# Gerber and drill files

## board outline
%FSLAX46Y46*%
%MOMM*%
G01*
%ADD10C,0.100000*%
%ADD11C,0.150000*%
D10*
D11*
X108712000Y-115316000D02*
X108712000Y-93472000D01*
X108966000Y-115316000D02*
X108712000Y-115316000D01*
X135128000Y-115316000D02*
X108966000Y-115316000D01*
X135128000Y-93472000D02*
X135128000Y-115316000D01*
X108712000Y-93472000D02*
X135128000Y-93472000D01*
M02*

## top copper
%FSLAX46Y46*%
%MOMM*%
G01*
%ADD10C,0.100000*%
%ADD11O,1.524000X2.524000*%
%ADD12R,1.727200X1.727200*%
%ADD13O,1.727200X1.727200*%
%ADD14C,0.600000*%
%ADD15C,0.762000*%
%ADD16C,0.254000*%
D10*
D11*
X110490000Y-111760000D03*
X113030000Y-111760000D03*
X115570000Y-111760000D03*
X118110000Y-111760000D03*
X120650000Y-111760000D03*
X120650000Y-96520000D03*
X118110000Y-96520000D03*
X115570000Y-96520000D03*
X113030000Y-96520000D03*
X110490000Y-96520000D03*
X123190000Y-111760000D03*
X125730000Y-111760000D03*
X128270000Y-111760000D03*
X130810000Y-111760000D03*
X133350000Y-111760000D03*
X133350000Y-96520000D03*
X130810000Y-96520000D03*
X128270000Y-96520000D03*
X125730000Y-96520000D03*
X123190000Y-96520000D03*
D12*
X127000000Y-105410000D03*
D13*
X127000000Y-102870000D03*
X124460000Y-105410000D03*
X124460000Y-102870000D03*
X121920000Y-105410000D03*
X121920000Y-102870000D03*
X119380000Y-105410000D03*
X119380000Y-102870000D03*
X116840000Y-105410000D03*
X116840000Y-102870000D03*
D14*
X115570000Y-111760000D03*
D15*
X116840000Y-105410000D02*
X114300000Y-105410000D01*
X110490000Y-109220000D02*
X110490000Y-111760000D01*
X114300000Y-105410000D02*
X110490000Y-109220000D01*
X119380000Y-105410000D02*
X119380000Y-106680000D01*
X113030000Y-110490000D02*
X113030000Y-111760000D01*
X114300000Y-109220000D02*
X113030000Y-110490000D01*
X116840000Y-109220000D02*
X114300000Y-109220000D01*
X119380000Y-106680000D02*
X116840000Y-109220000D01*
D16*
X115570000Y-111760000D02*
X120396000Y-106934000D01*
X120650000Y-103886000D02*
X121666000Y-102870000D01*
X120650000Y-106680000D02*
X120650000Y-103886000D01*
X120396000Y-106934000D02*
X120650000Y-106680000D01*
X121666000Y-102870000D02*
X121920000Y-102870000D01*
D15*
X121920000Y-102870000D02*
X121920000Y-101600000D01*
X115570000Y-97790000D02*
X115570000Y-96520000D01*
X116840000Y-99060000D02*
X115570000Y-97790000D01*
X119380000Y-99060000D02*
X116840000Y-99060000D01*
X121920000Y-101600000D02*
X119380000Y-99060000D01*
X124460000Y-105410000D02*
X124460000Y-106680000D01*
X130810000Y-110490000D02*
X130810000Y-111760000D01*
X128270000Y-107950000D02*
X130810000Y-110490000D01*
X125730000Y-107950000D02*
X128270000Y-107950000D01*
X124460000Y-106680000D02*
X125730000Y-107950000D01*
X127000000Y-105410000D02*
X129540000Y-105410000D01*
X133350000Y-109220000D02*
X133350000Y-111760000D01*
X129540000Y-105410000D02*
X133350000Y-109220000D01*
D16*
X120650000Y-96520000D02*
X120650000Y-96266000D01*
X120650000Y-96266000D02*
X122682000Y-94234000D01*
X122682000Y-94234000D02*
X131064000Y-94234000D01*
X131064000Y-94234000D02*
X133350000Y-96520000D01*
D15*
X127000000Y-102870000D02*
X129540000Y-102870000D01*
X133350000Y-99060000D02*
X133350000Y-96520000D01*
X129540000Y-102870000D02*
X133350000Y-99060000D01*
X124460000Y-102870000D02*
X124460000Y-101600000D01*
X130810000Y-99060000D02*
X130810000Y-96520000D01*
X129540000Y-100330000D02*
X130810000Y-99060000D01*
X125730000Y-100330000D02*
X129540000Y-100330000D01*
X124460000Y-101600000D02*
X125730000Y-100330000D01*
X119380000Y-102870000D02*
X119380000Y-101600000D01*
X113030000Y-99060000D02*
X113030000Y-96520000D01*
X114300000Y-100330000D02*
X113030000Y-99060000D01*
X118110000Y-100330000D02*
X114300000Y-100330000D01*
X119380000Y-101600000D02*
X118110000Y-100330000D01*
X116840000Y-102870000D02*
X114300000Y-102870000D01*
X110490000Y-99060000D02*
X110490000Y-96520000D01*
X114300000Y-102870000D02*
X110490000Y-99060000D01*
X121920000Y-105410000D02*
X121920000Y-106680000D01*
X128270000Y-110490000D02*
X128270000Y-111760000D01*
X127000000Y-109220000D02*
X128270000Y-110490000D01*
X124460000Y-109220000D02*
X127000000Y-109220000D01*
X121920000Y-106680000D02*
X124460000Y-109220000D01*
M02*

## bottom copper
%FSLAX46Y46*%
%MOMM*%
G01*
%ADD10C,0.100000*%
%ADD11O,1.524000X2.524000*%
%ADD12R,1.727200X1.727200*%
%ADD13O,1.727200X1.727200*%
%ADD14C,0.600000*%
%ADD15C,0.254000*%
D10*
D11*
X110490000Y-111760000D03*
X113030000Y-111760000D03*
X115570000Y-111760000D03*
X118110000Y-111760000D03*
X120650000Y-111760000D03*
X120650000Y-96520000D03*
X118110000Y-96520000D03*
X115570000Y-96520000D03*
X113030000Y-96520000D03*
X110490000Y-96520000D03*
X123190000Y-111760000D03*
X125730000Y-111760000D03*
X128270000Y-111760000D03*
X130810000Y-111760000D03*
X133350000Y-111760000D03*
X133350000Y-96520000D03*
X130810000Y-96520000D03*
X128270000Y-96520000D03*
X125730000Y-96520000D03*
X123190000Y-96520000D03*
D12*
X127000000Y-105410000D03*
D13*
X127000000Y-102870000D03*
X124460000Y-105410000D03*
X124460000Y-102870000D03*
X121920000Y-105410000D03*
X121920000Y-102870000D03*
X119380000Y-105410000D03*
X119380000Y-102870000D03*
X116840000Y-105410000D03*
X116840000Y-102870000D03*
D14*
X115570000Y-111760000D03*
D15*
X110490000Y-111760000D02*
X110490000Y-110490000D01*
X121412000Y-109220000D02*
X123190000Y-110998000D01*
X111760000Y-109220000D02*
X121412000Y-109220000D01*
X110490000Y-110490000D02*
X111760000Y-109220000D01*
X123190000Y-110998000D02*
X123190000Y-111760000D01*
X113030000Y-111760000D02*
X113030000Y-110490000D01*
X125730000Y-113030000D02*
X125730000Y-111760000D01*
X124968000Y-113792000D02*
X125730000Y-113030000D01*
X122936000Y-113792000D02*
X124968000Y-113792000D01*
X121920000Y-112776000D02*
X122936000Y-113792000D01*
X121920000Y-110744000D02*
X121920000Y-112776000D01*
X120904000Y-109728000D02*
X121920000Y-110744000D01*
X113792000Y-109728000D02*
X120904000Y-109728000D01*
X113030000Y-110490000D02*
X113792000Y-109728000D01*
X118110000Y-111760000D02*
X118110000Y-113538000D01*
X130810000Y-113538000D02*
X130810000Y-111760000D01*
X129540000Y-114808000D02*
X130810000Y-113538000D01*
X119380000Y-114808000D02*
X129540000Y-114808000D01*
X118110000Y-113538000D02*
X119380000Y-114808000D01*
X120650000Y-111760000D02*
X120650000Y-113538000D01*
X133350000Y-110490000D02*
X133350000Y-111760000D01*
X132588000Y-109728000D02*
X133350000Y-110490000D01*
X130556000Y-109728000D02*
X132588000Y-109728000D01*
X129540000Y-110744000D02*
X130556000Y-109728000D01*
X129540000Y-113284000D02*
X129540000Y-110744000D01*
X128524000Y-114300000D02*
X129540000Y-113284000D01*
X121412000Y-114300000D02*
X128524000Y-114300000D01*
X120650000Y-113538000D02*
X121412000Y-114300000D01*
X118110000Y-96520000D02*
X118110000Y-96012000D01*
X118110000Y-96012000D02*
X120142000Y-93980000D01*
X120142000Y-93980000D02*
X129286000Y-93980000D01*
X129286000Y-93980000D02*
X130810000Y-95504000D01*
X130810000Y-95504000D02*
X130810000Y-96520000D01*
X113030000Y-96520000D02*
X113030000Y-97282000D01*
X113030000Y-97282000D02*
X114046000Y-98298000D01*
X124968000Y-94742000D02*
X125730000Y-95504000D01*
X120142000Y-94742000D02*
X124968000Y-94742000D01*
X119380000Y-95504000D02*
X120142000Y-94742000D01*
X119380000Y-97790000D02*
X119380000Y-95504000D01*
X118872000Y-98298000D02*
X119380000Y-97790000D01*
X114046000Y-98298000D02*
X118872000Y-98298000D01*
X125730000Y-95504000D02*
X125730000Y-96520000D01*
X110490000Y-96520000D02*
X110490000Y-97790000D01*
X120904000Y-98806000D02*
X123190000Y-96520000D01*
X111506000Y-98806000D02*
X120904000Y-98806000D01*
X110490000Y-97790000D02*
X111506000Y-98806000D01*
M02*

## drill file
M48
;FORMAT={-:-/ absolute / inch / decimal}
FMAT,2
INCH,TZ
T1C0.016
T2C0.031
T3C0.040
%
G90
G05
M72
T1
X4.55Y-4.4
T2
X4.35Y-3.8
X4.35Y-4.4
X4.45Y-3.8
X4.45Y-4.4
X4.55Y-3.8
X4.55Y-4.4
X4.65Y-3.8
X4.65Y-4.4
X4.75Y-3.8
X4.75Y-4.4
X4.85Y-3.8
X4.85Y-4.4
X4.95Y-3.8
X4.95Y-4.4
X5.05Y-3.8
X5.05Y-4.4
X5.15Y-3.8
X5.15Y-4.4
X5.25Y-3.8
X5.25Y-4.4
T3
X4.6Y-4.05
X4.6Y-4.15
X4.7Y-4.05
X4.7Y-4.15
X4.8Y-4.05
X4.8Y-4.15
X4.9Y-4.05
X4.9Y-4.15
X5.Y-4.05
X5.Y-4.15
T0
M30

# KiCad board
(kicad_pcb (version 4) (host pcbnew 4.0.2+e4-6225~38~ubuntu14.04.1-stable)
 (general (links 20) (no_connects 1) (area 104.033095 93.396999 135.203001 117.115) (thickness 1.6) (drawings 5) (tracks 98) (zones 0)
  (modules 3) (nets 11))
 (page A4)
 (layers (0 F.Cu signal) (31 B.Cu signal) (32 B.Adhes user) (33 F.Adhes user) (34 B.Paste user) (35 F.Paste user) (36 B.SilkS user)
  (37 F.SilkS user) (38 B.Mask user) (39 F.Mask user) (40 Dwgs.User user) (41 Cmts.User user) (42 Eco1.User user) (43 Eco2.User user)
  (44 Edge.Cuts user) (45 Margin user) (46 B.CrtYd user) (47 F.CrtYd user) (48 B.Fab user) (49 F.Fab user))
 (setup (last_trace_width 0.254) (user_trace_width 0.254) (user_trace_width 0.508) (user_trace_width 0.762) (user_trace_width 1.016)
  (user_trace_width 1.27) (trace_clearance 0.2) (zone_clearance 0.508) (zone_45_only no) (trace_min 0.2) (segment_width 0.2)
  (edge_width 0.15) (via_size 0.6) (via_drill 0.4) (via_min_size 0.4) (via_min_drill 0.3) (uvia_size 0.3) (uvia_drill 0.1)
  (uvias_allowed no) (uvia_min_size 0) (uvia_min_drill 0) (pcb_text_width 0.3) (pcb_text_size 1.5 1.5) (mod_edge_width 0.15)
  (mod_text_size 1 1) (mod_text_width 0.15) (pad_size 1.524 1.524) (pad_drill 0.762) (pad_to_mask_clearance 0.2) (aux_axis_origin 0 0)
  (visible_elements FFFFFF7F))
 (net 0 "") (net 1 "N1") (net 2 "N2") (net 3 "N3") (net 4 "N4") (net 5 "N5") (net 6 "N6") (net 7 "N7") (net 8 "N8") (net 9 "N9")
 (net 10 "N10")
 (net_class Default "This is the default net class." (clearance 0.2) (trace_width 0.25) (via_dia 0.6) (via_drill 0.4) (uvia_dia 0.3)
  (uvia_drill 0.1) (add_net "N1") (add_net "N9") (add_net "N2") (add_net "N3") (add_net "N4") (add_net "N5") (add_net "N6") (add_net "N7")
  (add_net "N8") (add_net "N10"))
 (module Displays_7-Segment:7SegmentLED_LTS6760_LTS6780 (layer F.Cu) (at 115.57 104.14)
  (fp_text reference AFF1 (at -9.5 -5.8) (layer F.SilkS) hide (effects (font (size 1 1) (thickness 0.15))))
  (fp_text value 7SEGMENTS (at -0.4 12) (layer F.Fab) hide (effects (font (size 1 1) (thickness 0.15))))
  (pad 1 thru_hole oval (at -5.08 7.62) (size 1.524 2.524) (drill 0.8) (layers *.Cu *.Mask F.SilkS) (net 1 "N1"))
  (pad 2 thru_hole oval (at -2.54 7.62) (size 1.524 2.524) (drill 0.8) (layers *.Cu *.Mask F.SilkS) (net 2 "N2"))
  (pad 3 thru_hole oval (at 0 7.62) (size 1.524 2.524) (drill 0.8) (layers *.Cu *.Mask F.SilkS) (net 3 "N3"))
  (pad 4 thru_hole oval (at 2.54 7.62) (size 1.524 2.524) (drill 0.8) (layers *.Cu *.Mask F.SilkS) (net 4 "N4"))
  (pad 5 thru_hole oval (at 5.08 7.62) (size 1.524 2.524) (drill 0.8) (layers *.Cu *.Mask F.SilkS) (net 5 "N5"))
  (pad 6 thru_hole oval (at 5.08 -7.62) (size 1.524 2.524) (drill 0.8) (layers *.Cu *.Mask F.SilkS) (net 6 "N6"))
  (pad 7 thru_hole oval (at 2.54 -7.62) (size 1.524 2.524) (drill 0.8) (layers *.Cu *.Mask F.SilkS) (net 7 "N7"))
  (pad 8 thru_hole oval (at 0 -7.62) (size 1.524 2.524) (drill 0.8) (layers *.Cu *.Mask F.SilkS) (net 3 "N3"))
  (pad 9 thru_hole oval (at -2.54 -7.62) (size 1.524 2.524) (drill 0.8) (layers *.Cu *.Mask F.SilkS) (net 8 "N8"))
  (pad 10 thru_hole oval (at -5.08 -7.62) (size 1.524 2.524) (drill 0.8) (layers *.Cu *.Mask F.SilkS) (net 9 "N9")))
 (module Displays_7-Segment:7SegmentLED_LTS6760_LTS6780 (layer F.Cu) (at 128.27 104.14)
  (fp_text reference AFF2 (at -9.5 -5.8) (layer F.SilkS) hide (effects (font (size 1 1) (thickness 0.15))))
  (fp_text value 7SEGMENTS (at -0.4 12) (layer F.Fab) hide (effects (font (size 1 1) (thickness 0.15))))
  (pad 1 thru_hole oval (at -5.08 7.62) (size 1.524 2.524) (drill 0.8) (layers *.Cu *.Mask F.SilkS) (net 1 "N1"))
  (pad 2 thru_hole oval (at -2.54 7.62) (size 1.524 2.524) (drill 0.8) (layers *.Cu *.Mask F.SilkS) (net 2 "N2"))
  (pad 3 thru_hole oval (at 0 7.62) (size 1.524 2.524) (drill 0.8) (layers *.Cu *.Mask F.SilkS) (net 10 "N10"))
  (pad 4 thru_hole oval (at 2.54 7.62) (size 1.524 2.524) (drill 0.8) (layers *.Cu *.Mask F.SilkS) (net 4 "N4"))
  (pad 5 thru_hole oval (at 5.08 7.62) (size 1.524 2.524) (drill 0.8) (layers *.Cu *.Mask F.SilkS) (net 5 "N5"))
  (pad 6 thru_hole oval (at 5.08 -7.62) (size 1.524 2.524) (drill 0.8) (layers *.Cu *.Mask F.SilkS) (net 6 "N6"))
  (pad 7 thru_hole oval (at 2.54 -7.62) (size 1.524 2.524) (drill 0.8) (layers *.Cu *.Mask F.SilkS) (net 7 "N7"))
  (pad 8 thru_hole oval (at 0 -7.62) (size 1.524 2.524) (drill 0.8) (layers *.Cu *.Mask F.SilkS) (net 10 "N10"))
  (pad 9 thru_hole oval (at -2.54 -7.62) (size 1.524 2.524) (drill 0.8) (layers *.Cu *.Mask F.SilkS) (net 8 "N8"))
  (pad 10 thru_hole oval (at -5.08 -7.62) (size 1.524 2.524) (drill 0.8) (layers *.Cu *.Mask F.SilkS) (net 9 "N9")))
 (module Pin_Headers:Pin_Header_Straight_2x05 (layer B.Cu) (at 127 105.41 90)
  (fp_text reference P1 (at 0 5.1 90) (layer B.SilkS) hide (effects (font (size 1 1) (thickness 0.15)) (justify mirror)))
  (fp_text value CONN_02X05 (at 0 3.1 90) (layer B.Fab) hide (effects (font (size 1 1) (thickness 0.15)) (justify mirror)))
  (pad 1 thru_hole rect (at 0 0 90) (size 1.7272 1.7272) (drill 1.016) (layers *.Cu *.Mask B.SilkS) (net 5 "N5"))
  (pad 2 thru_hole oval (at 2.54 0 90) (size 1.7272 1.7272) (drill 1.016) (layers *.Cu *.Mask B.SilkS) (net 6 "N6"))
  (pad 3 thru_hole oval (at 0 -2.54 90) (size 1.7272 1.7272) (drill 1.016) (layers *.Cu *.Mask B.SilkS) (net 4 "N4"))
  (pad 4 thru_hole oval (at 2.54 -2.54 90) (size 1.7272 1.7272) (drill 1.016) (layers *.Cu *.Mask B.SilkS) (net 7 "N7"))
  (pad 5 thru_hole oval (at 0 -5.08 90) (size 1.7272 1.7272) (drill 1.016) (layers *.Cu *.Mask B.SilkS) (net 10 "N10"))
  (pad 6 thru_hole oval (at 2.54 -5.08 90) (size 1.7272 1.7272) (drill 1.016) (layers *.Cu *.Mask B.SilkS) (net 3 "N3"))
  (pad 7 thru_hole oval (at 0 -7.62 90) (size 1.7272 1.7272) (drill 1.016) (layers *.Cu *.Mask B.SilkS) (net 2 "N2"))
  (pad 8 thru_hole oval (at 2.54 -7.62 90) (size 1.7272 1.7272) (drill 1.016) (layers *.Cu *.Mask B.SilkS) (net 8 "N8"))
  (pad 9 thru_hole oval (at 0 -10.16 90) (size 1.7272 1.7272) (drill 1.016) (layers *.Cu *.Mask B.SilkS) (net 1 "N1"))
  (pad 10 thru_hole oval (at 2.54 -10.16 90) (size 1.7272 1.7272) (drill 1.016) (layers *.Cu *.Mask B.SilkS) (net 9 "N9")))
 (gr_line (start 108.712 115.316) (end 108.712 93.472) (angle 90) (layer Edge.Cuts) (width 0.15))
 (gr_line (start 108.966 115.316) (end 108.712 115.316) (angle 90) (layer Edge.Cuts) (width 0.15))
 (gr_line (start 135.128 115.316) (end 108.966 115.316) (angle 90) (layer Edge.Cuts) (width 0.15))
 (gr_line (start 135.128 93.472) (end 135.128 115.316) (angle 90) (layer Edge.Cuts) (width 0.15))
 (gr_line (start 108.712 93.472) (end 135.128 93.472) (angle 90) (layer Edge.Cuts) (width 0.15))
 (segment (start 110.49 111.76) (end 110.49 110.49) (width 0.254) (layer B.Cu) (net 1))
 (segment (start 121.412 109.22) (end 123.19 110.998) (width 0.254) (layer B.Cu) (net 1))
 (segment (start 111.76 109.22) (end 121.412 109.22) (width 0.254) (layer B.Cu) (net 1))
 (segment (start 110.49 110.49) (end 111.76 109.22) (width 0.254) (layer B.Cu) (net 1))
 (segment (start 123.19 110.998) (end 123.19 111.76) (width 0.254) (layer B.Cu) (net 1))
 (segment (start 116.84 105.41) (end 114.3 105.41) (width 0.762) (layer F.Cu) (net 1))
 (segment (start 110.49 109.22) (end 110.49 111.76) (width 0.762) (layer F.Cu) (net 1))
 (segment (start 114.3 105.41) (end 110.49 109.22) (width 0.762) (layer F.Cu) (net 1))
 (segment (start 113.03 111.76) (end 113.03 110.49) (width 0.254) (layer B.Cu) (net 2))
 (segment (start 125.73 113.03) (end 125.73 111.76) (width 0.254) (layer B.Cu) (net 2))
 (segment (start 124.968 113.792) (end 125.73 113.03) (width 0.254) (layer B.Cu) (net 2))
 (segment (start 122.936 113.792) (end 124.968 113.792) (width 0.254) (layer B.Cu) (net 2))
 (segment (start 121.92 112.776) (end 122.936 113.792) (width 0.254) (layer B.Cu) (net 2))
 (segment (start 121.92 110.744) (end 121.92 112.776) (width 0.254) (layer B.Cu) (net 2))
 (segment (start 120.904 109.728) (end 121.92 110.744) (width 0.254) (layer B.Cu) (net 2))
 (segment (start 113.792 109.728) (end 120.904 109.728) (width 0.254) (layer B.Cu) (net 2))
 (segment (start 113.03 110.49) (end 113.792 109.728) (width 0.254) (layer B.Cu) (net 2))
 (segment (start 119.38 105.41) (end 119.38 106.68) (width 0.762) (layer F.Cu) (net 2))
 (segment (start 113.03 110.49) (end 113.03 111.76) (width 0.762) (layer F.Cu) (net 2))
 (segment (start 114.3 109.22) (end 113.03 110.49) (width 0.762) (layer F.Cu) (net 2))
 (segment (start 116.84 109.22) (end 114.3 109.22) (width 0.762) (layer F.Cu) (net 2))
 (segment (start 119.38 106.68) (end 116.84 109.22) (width 0.762) (layer F.Cu) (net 2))
 (via (at 115.57 111.76) (size 0.6) (drill 0.4) (layers F.Cu B.Cu) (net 3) (status C00000))
 (segment (start 115.57 111.76) (end 120.396 106.934) (width 0.254) (layer F.Cu) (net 3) (status 400000))
 (segment (start 120.65 103.886) (end 121.666 102.87) (width 0.254) (layer F.Cu) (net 3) (status 800000))
 (segment (start 120.65 106.68) (end 120.65 103.886) (width 0.254) (layer F.Cu) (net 3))
 (segment (start 120.396 106.934) (end 120.65 106.68) (width 0.254) (layer F.Cu) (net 3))
 (segment (start 121.666 102.87) (end 121.92 102.87) (width 0.254) (layer F.Cu) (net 3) (status C00000))
 (segment (start 121.92 102.87) (end 121.92 101.6) (width 0.762) (layer F.Cu) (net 3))
 (segment (start 115.57 97.79) (end 115.57 96.52) (width 0.762) (layer F.Cu) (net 3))
 (segment (start 116.84 99.06) (end 115.57 97.79) (width 0.762) (layer F.Cu) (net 3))
 (segment (start 119.38 99.06) (end 116.84 99.06) (width 0.762) (layer F.Cu) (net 3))
 (segment (start 121.92 101.6) (end 119.38 99.06) (width 0.762) (layer F.Cu) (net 3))
 (segment (start 118.11 111.76) (end 118.11 113.538) (width 0.254) (layer B.Cu) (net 4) (status 400000))
 (segment (start 130.81 113.538) (end 130.81 111.76) (width 0.254) (layer B.Cu) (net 4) (status 800000))
 (segment (start 129.54 114.808) (end 130.81 113.538) (width 0.254) (layer B.Cu) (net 4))
 (segment (start 119.38 114.808) (end 129.54 114.808) (width 0.254) (layer B.Cu) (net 4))
 (segment (start 118.11 113.538) (end 119.38 114.808) (width 0.254) (layer B.Cu) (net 4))
 (segment (start 124.46 105.41) (end 124.46 106.68) (width 0.762) (layer F.Cu) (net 4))
 (segment (start 130.81 110.49) (end 130.81 111.76) (width 0.762) (layer F.Cu) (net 4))
 (segment (start 128.27 107.95) (end 130.81 110.49) (width 0.762) (layer F.Cu) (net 4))
 (segment (start 125.73 107.95) (end 128.27 107.95) (width 0.762) (layer F.Cu) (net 4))
 (segment (start 124.46 106.68) (end 125.73 107.95) (width 0.762) (layer F.Cu) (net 4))
 (segment (start 120.65 111.76) (end 120.65 113.538) (width 0.254) (layer B.Cu) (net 5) (status 400000))
 (segment (start 133.35 110.49) (end 133.35 111.76) (width 0.254) (layer B.Cu) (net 5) (status 800000))
 (segment (start 132.588 109.728) (end 133.35 110.49) (width 0.254) (layer B.Cu) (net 5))
 (segment (start 130.556 109.728) (end 132.588 109.728) (width 0.254) (layer B.Cu) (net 5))
 (segment (start 129.54 110.744) (end 130.556 109.728) (width 0.254) (layer B.Cu) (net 5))
 (segment (start 129.54 113.284) (end 129.54 110.744) (width 0.254) (layer B.Cu) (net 5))
 (segment (start 128.524 114.3) (end 129.54 113.284) (width 0.254) (layer B.Cu) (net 5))
 (segment (start 121.412 114.3) (end 128.524 114.3) (width 0.254) (layer B.Cu) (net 5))
 (segment (start 120.65 113.538) (end 121.412 114.3) (width 0.254) (layer B.Cu) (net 5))
 (segment (start 127 105.41) (end 129.54 105.41) (width 0.762) (layer F.Cu) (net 5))
 (segment (start 133.35 109.22) (end 133.35 111.76) (width 0.762) (layer F.Cu) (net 5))
 (segment (start 129.54 105.41) (end 133.35 109.22) (width 0.762) (layer F.Cu) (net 5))
 (segment (start 120.65 96.52) (end 120.65 96.266) (width 0.254) (layer F.Cu) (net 6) (status C00000))
 (segment (start 120.65 96.266) (end 122.682 94.234) (width 0.254) (layer F.Cu) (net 6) (status 400000))
 (segment (start 122.682 94.234) (end 131.064 94.234) (width 0.254) (layer F.Cu) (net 6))
 (segment (start 131.064 94.234) (end 133.35 96.52) (width 0.254) (layer F.Cu) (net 6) (status 800000))
 (segment (start 127 102.87) (end 129.54 102.87) (width 0.762) (layer F.Cu) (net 6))
 (segment (start 133.35 99.06) (end 133.35 96.52) (width 0.762) (layer F.Cu) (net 6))
 (segment (start 129.54 102.87) (end 133.35 99.06) (width 0.762) (layer F.Cu) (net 6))
 (segment (start 118.11 96.52) (end 118.11 96.012) (width 0.254) (layer B.Cu) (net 7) (status C00000))
 (segment (start 118.11 96.012) (end 120.142 93.98) (width 0.254) (layer B.Cu) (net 7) (status 400000))
 (segment (start 120.142 93.98) (end 129.286 93.98) (width 0.254) (layer B.Cu) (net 7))
 (segment (start 129.286 93.98) (end 130.81 95.504) (width 0.254) (layer B.Cu) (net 7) (status 800000))
 (segment (start 130.81 95.504) (end 130.81 96.52) (width 0.254) (layer B.Cu) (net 7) (status C00000))
 (segment (start 124.46 102.87) (end 124.46 101.6) (width 0.762) (layer F.Cu) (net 7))
 (segment (start 130.81 99.06) (end 130.81 96.52) (width 0.762) (layer F.Cu) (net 7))
 (segment (start 129.54 100.33) (end 130.81 99.06) (width 0.762) (layer F.Cu) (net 7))
 (segment (start 125.73 100.33) (end 129.54 100.33) (width 0.762) (layer F.Cu) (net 7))
 (segment (start 124.46 101.6) (end 125.73 100.33) (width 0.762) (layer F.Cu) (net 7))
 (segment (start 113.03 96.52) (end 113.03 97.282) (width 0.254) (layer B.Cu) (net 8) (status C00000))
 (segment (start 113.03 97.282) (end 114.046 98.298) (width 0.254) (layer B.Cu) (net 8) (status 400000))
 (segment (start 124.968 94.742) (end 125.73 95.504) (width 0.254) (layer B.Cu) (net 8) (status 800000))
 (segment (start 120.142 94.742) (end 124.968 94.742) (width 0.254) (layer B.Cu) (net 8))
 (segment (start 119.38 95.504) (end 120.142 94.742) (width 0.254) (layer B.Cu) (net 8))
 (segment (start 119.38 97.79) (end 119.38 95.504) (width 0.254) (layer B.Cu) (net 8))
 (segment (start 118.872 98.298) (end 119.38 97.79) (width 0.254) (layer B.Cu) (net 8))
 (segment (start 114.046 98.298) (end 118.872 98.298) (width 0.254) (layer B.Cu) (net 8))
 (segment (start 125.73 95.504) (end 125.73 96.52) (width 0.254) (layer B.Cu) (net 8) (status C00000))
 (segment (start 119.38 102.87) (end 119.38 101.6) (width 0.762) (layer F.Cu) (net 8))
 (segment (start 113.03 99.06) (end 113.03 96.52) (width 0.762) (layer F.Cu) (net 8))
 (segment (start 114.3 100.33) (end 113.03 99.06) (width 0.762) (layer F.Cu) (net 8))
 (segment (start 118.11 100.33) (end 114.3 100.33) (width 0.762) (layer F.Cu) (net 8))
 (segment (start 119.38 101.6) (end 118.11 100.33) (width 0.762) (layer F.Cu) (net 8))
 (segment (start 110.49 96.52) (end 110.49 97.79) (width 0.254) (layer B.Cu) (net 9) (status 400000))
 (segment (start 120.904 98.806) (end 123.19 96.52) (width 0.254) (layer B.Cu) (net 9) (status 800000))
 (segment (start 111.506 98.806) (end 120.904 98.806) (width 0.254) (layer B.Cu) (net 9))
 (segment (start 110.49 97.79) (end 111.506 98.806) (width 0.254) (layer B.Cu) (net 9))
 (segment (start 116.84 102.87) (end 114.3 102.87) (width 0.762) (layer F.Cu) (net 9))
 (segment (start 110.49 99.06) (end 110.49 96.52) (width 0.762) (layer F.Cu) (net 9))
 (segment (start 114.3 102.87) (end 110.49 99.06) (width 0.762) (layer F.Cu) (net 9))
 (segment (start 121.92 105.41) (end 121.92 106.68) (width 0.762) (layer F.Cu) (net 10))
 (segment (start 128.27 110.49) (end 128.27 111.76) (width 0.762) (layer F.Cu) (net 10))
 (segment (start 127 109.22) (end 128.27 110.49) (width 0.762) (layer F.Cu) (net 10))
 (segment (start 124.46 109.22) (end 127 109.22) (width 0.762) (layer F.Cu) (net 10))
 (segment (start 121.92 106.68) (end 124.46 109.22) (width 0.762) (layer F.Cu) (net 10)))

